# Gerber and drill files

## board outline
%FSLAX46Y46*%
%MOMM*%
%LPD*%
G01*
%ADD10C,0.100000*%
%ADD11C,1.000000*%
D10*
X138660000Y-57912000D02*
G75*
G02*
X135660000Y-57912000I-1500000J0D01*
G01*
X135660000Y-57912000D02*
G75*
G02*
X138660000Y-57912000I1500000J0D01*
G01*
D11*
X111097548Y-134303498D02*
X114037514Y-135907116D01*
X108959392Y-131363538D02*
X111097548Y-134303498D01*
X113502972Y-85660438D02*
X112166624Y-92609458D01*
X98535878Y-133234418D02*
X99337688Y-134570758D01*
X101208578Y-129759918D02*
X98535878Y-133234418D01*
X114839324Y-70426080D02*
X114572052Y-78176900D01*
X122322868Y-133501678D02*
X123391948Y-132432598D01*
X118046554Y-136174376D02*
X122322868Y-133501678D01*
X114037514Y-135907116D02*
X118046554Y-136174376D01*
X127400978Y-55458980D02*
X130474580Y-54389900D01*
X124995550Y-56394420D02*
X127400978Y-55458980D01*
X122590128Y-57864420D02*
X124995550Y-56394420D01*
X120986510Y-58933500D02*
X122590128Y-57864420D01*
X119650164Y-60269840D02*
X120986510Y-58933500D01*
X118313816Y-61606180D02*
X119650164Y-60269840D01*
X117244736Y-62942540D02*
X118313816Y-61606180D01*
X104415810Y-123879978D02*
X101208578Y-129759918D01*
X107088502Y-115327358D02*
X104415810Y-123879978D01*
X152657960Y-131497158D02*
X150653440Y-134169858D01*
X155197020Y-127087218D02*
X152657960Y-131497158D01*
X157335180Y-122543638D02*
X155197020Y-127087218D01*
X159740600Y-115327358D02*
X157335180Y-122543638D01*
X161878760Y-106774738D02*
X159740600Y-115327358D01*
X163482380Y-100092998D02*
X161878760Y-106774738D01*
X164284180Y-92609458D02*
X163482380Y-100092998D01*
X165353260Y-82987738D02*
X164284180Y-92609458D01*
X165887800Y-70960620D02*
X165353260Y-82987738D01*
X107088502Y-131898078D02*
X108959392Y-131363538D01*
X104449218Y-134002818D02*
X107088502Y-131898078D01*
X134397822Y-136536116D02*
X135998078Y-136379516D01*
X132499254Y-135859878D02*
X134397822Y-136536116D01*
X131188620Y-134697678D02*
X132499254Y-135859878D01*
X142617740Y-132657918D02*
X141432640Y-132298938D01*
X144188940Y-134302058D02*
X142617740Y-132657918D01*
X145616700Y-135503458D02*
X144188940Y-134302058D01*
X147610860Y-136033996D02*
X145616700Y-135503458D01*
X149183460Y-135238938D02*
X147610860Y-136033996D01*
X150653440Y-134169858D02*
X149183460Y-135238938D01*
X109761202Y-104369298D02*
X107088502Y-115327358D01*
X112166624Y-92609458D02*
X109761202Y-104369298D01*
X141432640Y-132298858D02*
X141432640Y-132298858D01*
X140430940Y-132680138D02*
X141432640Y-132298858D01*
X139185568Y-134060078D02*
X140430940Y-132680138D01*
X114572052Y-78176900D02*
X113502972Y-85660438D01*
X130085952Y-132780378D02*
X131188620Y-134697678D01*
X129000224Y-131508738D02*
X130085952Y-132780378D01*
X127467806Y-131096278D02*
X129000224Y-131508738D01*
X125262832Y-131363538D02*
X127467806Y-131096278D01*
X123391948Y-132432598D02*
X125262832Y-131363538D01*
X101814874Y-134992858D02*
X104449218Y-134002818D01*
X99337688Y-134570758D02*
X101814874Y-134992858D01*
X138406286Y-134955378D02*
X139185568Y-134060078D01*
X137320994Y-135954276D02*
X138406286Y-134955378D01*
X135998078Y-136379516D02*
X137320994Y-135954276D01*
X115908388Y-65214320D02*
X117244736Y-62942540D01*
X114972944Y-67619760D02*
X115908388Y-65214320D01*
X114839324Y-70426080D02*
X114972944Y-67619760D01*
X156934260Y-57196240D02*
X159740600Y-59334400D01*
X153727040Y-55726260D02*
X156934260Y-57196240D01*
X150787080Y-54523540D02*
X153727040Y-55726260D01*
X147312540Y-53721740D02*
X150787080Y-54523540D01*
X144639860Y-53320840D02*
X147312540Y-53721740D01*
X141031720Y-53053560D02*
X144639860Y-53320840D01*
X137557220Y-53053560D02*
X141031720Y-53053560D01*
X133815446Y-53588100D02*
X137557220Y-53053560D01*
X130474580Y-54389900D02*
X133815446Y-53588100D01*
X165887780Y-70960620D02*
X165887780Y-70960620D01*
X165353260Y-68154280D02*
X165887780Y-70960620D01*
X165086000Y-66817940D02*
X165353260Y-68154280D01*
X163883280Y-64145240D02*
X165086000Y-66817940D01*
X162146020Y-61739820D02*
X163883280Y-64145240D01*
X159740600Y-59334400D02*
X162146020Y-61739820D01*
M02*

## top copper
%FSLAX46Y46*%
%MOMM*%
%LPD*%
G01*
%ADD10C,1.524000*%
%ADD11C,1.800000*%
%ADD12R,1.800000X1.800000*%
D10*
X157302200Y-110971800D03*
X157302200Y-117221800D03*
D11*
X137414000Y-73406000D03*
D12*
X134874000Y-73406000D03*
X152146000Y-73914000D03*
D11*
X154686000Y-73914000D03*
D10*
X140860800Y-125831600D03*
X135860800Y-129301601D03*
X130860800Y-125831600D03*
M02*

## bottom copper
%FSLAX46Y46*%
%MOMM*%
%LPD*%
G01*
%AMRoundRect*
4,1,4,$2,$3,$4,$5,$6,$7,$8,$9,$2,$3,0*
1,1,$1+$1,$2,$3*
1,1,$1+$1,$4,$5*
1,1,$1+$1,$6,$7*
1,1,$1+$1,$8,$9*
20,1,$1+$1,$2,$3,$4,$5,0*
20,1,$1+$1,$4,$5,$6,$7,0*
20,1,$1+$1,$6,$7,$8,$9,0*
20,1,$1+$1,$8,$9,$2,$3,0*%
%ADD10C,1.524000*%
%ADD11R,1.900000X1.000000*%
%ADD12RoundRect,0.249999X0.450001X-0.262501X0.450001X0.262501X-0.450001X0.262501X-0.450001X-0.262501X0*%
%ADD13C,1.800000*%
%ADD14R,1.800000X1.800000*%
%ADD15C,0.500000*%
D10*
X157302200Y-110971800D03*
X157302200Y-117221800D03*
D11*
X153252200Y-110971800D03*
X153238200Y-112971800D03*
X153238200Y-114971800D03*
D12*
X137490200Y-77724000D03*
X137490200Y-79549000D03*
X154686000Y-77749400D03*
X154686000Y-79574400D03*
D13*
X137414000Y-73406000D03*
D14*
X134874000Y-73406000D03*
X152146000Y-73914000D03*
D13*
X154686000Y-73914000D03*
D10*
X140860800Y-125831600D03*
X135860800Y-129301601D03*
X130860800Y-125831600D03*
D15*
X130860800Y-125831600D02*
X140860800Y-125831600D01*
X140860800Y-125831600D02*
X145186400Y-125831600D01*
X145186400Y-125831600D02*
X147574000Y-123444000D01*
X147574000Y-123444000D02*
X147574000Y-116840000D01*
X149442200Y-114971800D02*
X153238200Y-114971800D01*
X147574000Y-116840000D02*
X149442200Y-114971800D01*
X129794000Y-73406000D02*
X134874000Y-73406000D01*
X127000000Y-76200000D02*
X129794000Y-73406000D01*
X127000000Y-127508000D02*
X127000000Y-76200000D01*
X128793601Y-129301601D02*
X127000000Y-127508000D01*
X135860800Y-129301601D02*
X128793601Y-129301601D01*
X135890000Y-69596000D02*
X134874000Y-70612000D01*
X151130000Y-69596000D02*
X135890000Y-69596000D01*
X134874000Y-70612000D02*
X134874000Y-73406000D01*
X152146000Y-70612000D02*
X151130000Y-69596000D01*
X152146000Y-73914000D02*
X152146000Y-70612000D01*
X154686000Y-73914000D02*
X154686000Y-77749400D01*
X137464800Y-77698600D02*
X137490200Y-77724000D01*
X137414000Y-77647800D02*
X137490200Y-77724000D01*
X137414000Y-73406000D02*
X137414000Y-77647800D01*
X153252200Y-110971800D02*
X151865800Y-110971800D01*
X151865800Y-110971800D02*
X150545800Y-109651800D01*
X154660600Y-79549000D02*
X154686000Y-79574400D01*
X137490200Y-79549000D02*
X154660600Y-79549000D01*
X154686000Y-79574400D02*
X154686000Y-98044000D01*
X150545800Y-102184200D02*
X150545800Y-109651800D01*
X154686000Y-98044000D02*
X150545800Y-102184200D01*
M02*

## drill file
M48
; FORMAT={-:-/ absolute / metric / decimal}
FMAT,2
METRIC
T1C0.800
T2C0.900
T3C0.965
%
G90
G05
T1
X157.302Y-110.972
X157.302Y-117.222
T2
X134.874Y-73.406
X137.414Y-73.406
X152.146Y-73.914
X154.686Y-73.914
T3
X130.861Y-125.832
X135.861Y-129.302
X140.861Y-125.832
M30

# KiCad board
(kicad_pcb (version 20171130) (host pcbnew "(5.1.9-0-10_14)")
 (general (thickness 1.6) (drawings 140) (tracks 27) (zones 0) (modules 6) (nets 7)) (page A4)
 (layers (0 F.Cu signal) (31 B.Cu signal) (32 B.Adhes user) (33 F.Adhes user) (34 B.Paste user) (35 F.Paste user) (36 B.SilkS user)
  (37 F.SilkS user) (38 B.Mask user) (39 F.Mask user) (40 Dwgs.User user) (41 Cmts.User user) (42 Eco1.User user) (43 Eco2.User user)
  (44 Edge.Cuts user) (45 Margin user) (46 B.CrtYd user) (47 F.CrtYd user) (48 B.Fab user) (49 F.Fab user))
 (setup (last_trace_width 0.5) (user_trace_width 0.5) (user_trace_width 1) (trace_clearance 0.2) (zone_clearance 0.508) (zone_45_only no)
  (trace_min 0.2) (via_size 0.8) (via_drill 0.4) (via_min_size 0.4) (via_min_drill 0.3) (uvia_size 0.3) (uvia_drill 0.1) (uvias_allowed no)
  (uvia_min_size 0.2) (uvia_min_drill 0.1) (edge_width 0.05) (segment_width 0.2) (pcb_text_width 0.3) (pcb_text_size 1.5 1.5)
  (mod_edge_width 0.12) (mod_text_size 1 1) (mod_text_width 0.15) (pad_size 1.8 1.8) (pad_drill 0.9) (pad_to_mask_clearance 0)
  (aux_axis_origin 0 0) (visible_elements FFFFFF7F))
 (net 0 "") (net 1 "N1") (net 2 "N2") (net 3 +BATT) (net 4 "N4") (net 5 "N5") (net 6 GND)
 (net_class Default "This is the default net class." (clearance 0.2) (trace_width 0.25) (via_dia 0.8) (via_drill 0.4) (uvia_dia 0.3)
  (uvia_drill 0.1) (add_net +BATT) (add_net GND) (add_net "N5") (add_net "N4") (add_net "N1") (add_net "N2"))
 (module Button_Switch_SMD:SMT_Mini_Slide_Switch (layer B.Cu) (at 155.0162 114.0968 270)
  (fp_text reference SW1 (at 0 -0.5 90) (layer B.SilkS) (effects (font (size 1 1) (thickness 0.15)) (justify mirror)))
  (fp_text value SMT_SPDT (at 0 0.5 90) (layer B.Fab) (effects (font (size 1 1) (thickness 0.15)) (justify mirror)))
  (pad "" thru_hole circle (at -3.125 -2.286 270) (size 1.524 1.524) (drill 0.8) (layers *.Cu *.Mask))
  (pad "" thru_hole circle (at 3.125 -2.286 270) (size 1.524 1.524) (drill 0.8) (layers *.Cu *.Mask))
  (pad 1 smd rect (at -3.125 1.764 270) (size 1 1.9) (layers B.Cu B.Paste B.Mask) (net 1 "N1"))
  (pad 2 smd rect (at -1.125 1.778 270) (size 1 1.9) (layers B.Cu B.Paste B.Mask) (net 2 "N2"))
  (pad 3 smd rect (at 0.875 1.778 270) (size 1 1.9) (layers B.Cu B.Paste B.Mask) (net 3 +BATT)))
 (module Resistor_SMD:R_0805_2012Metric (layer B.Cu) (at 137.4902 78.6365 90)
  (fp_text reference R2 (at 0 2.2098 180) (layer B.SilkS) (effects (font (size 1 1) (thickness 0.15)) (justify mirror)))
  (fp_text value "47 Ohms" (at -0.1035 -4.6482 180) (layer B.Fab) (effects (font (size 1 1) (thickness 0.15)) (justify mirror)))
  (pad 2 smd roundrect (at 0.9125 0 90) (size 1.025 1.4) (layers B.Cu B.Paste B.Mask) (roundrect_rratio 0.2439014634146341) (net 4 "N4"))
  (pad 1 smd roundrect (at -0.9125 0 90) (size 1.025 1.4) (layers B.Cu B.Paste B.Mask) (roundrect_rratio 0.2439014634146341) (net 1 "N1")))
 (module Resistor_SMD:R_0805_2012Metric (layer B.Cu) (at 154.686 78.6619 90)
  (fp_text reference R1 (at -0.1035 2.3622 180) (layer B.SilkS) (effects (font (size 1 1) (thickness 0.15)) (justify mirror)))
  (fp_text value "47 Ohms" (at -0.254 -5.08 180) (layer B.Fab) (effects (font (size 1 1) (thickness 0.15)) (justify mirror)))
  (pad 2 smd roundrect (at 0.9125 0 90) (size 1.025 1.4) (layers B.Cu B.Paste B.Mask) (roundrect_rratio 0.2439014634146341) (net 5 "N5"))
  (pad 1 smd roundrect (at -0.9125 0 90) (size 1.025 1.4) (layers B.Cu B.Paste B.Mask) (roundrect_rratio 0.2439014634146341) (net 1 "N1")))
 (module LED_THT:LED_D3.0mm (layer F.Cu) (at 134.874 73.406)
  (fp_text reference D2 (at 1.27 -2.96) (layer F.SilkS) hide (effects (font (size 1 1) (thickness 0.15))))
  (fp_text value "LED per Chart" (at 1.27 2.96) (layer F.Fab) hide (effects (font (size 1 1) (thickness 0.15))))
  (pad 2 thru_hole circle (at 2.54 0) (size 1.8 1.8) (drill 0.9) (layers *.Cu *.Mask) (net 4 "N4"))
  (pad 1 thru_hole rect (at 0 0) (size 1.8 1.8) (drill 0.9) (layers *.Cu *.Mask) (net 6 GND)))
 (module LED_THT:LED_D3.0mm (layer F.Cu) (at 152.146 73.914)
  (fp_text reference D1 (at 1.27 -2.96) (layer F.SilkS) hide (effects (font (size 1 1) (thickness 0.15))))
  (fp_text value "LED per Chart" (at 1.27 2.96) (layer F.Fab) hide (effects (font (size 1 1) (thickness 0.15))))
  (pad 1 thru_hole rect (at 0 0) (size 1.8 1.8) (drill 0.9) (layers *.Cu *.Mask) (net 6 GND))
  (pad 2 thru_hole circle (at 2.54 0) (size 1.8 1.8) (drill 0.9) (layers *.Cu *.Mask) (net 5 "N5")))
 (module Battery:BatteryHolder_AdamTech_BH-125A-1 (layer B.Cu) (at 130.8608 125.8316)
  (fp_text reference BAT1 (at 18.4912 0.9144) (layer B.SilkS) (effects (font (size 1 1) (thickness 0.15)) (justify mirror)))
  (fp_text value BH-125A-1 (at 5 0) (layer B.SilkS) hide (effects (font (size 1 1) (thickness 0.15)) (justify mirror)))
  (pad POS2 thru_hole circle (at 10 0) (size 1.524 1.524) (drill 0.9652) (layers *.Cu *.Mask) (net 3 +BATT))
  (pad NEG thru_hole circle (at 5 3.470001) (size 1.524 1.524) (drill 0.9652) (layers *.Cu *.Mask) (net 6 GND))
  (pad POS1 thru_hole circle (at 0 0) (size 1.524 1.524) (drill 0.9652) (layers *.Cu *.Mask) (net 3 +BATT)))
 (gr_circle (center 137.16 57.912) (end 138.66 57.912) (layer Edge.Cuts) (width 0.1))
 (gr_line (start 111.097548 134.303498) (end 114.037514 135.907116) (layer Edge.Cuts) (width 1))
 (gr_line (start 108.959392 131.363538) (end 111.097548 134.303498) (layer Edge.Cuts) (width 1))
 (gr_line (start 113.502972 85.660438) (end 112.166624 92.609458) (layer Edge.Cuts) (width 1))
 (gr_line (start 98.535878 133.234418) (end 99.337688 134.570758) (layer Edge.Cuts) (width 1))
 (gr_line (start 101.208578 129.759918) (end 98.535878 133.234418) (layer Edge.Cuts) (width 1))
 (gr_line (start 114.839324 70.42608) (end 114.572052 78.1769) (layer Edge.Cuts) (width 1))
 (gr_line (start 122.322868 133.501678) (end 123.391948 132.432598) (layer Edge.Cuts) (width 1))
 (gr_line (start 118.046554 136.174376) (end 122.322868 133.501678) (layer Edge.Cuts) (width 1))
 (gr_line (start 114.037514 135.907116) (end 118.046554 136.174376) (layer Edge.Cuts) (width 1))
 (gr_line (start 127.400978 55.45898) (end 130.47458 54.3899) (layer Edge.Cuts) (width 1))
 (gr_line (start 124.99555 56.39442) (end 127.400978 55.45898) (layer Edge.Cuts) (width 1))
 (gr_line (start 122.590128 57.86442) (end 124.99555 56.39442) (layer Edge.Cuts) (width 1))
 (gr_line (start 120.98651 58.9335) (end 122.590128 57.86442) (layer Edge.Cuts) (width 1))
 (gr_line (start 119.650164 60.26984) (end 120.98651 58.9335) (layer Edge.Cuts) (width 1))
 (gr_line (start 118.313816 61.60618) (end 119.650164 60.26984) (layer Edge.Cuts) (width 1))
 (gr_line (start 117.244736 62.94254) (end 118.313816 61.60618) (layer Edge.Cuts) (width 1))
 (gr_line (start 104.41581 123.879978) (end 101.208578 129.759918) (layer Edge.Cuts) (width 1))
 (gr_line (start 107.088502 115.327358) (end 104.41581 123.879978) (layer Edge.Cuts) (width 1))
 (gr_line (start 152.65796 131.497158) (end 150.65344 134.169858) (layer Edge.Cuts) (width 1))
 (gr_line (start 155.19702 127.087218) (end 152.65796 131.497158) (layer Edge.Cuts) (width 1))
 (gr_line (start 157.33518 122.543638) (end 155.19702 127.087218) (layer Edge.Cuts) (width 1))
 (gr_line (start 159.7406 115.327358) (end 157.33518 122.543638) (layer Edge.Cuts) (width 1))
 (gr_line (start 161.87876 106.774738) (end 159.7406 115.327358) (layer Edge.Cuts) (width 1))
 (gr_line (start 163.48238 100.092998) (end 161.87876 106.774738) (layer Edge.Cuts) (width 1))
 (gr_line (start 164.28418 92.609458) (end 163.48238 100.092998) (layer Edge.Cuts) (width 1))
 (gr_line (start 165.35326 82.987738) (end 164.28418 92.609458) (layer Edge.Cuts) (width 1))
 (gr_line (start 165.8878 70.96062) (end 165.35326 82.987738) (layer Edge.Cuts) (width 1))
 (gr_line (start 107.088502 131.898078) (end 108.959392 131.363538) (layer Edge.Cuts) (width 1))
 (gr_line (start 104.449218 134.002818) (end 107.088502 131.898078) (layer Edge.Cuts) (width 1))
 (gr_line (start 134.397822 136.536116) (end 135.998078 136.379516) (layer Edge.Cuts) (width 1))
 (gr_line (start 132.499254 135.859878) (end 134.397822 136.536116) (layer Edge.Cuts) (width 1))
 (gr_line (start 131.18862 134.697678) (end 132.499254 135.859878) (layer Edge.Cuts) (width 1))
 (gr_line (start 142.61774 132.657918) (end 141.43264 132.298938) (layer Edge.Cuts) (width 1))
 (gr_line (start 144.18894 134.302058) (end 142.61774 132.657918) (layer Edge.Cuts) (width 1))
 (gr_line (start 145.6167 135.503458) (end 144.18894 134.302058) (layer Edge.Cuts) (width 1))
 (gr_line (start 147.61086 136.033996) (end 145.6167 135.503458) (layer Edge.Cuts) (width 1))
 (gr_line (start 149.18346 135.238938) (end 147.61086 136.033996) (layer Edge.Cuts) (width 1))
 (gr_line (start 150.65344 134.169858) (end 149.18346 135.238938) (layer Edge.Cuts) (width 1))
 (gr_line (start 109.761202 104.369298) (end 107.088502 115.327358) (layer Edge.Cuts) (width 1))
 (gr_line (start 112.166624 92.609458) (end 109.761202 104.369298) (layer Edge.Cuts) (width 1))
 (gr_line (start 141.43264 132.298858) (end 141.43264 132.298858) (layer Edge.Cuts) (width 1))
 (gr_line (start 140.43094 132.680138) (end 141.43264 132.298858) (layer Edge.Cuts) (width 1))
 (gr_line (start 139.185568 134.060078) (end 140.43094 132.680138) (layer Edge.Cuts) (width 1))
 (gr_line (start 114.572052 78.1769) (end 113.502972 85.660438) (layer Edge.Cuts) (width 1))
 (gr_line (start 130.085952 132.780378) (end 131.18862 134.697678) (layer Edge.Cuts) (width 1))
 (gr_line (start 129.000224 131.508738) (end 130.085952 132.780378) (layer Edge.Cuts) (width 1))
 (gr_line (start 127.467806 131.096278) (end 129.000224 131.508738) (layer Edge.Cuts) (width 1))
 (gr_line (start 125.262832 131.363538) (end 127.467806 131.096278) (layer Edge.Cuts) (width 1))
 (gr_line (start 123.391948 132.432598) (end 125.262832 131.363538) (layer Edge.Cuts) (width 1))
 (gr_line (start 101.814874 134.992858) (end 104.449218 134.002818) (layer Edge.Cuts) (width 1))
 (gr_line (start 99.337688 134.570758) (end 101.814874 134.992858) (layer Edge.Cuts) (width 1))
 (gr_line (start 138.406286 134.955378) (end 139.185568 134.060078) (layer Edge.Cuts) (width 1))
 (gr_line (start 137.320994 135.954276) (end 138.406286 134.955378) (layer Edge.Cuts) (width 1))
 (gr_line (start 135.998078 136.379516) (end 137.320994 135.954276) (layer Edge.Cuts) (width 1))
 (gr_line (start 115.908388 65.21432) (end 117.244736 62.94254) (layer Edge.Cuts) (width 1))
 (gr_line (start 114.972944 67.61976) (end 115.908388 65.21432) (layer Edge.Cuts) (width 1))
 (gr_line (start 114.839324 70.42608) (end 114.972944 67.61976) (layer Edge.Cuts) (width 1))
 (gr_line (start 156.93426 57.19624) (end 159.7406 59.3344) (layer Edge.Cuts) (width 1))
 (gr_line (start 153.72704 55.72626) (end 156.93426 57.19624) (layer Edge.Cuts) (width 1))
 (gr_line (start 150.78708 54.52354) (end 153.72704 55.72626) (layer Edge.Cuts) (width 1))
 (gr_line (start 147.31254 53.72174) (end 150.78708 54.52354) (layer Edge.Cuts) (width 1))
 (gr_line (start 144.63986 53.32084) (end 147.31254 53.72174) (layer Edge.Cuts) (width 1))
 (gr_line (start 141.03172 53.05356) (end 144.63986 53.32084) (layer Edge.Cuts) (width 1))
 (gr_line (start 137.55722 53.05356) (end 141.03172 53.05356) (layer Edge.Cuts) (width 1))
 (gr_line (start 133.815446 53.5881) (end 137.55722 53.05356) (layer Edge.Cuts) (width 1))
 (gr_line (start 130.47458 54.3899) (end 133.815446 53.5881) (layer Edge.Cuts) (width 1))
 (gr_line (start 165.88778 70.96062) (end 165.88778 70.96062) (layer Edge.Cuts) (width 1))
 (gr_line (start 165.35326 68.15428) (end 165.88778 70.96062) (layer Edge.Cuts) (width 1))
 (gr_line (start 165.086 66.81794) (end 165.35326 68.15428) (layer Edge.Cuts) (width 1))
 (gr_line (start 163.88328 64.14524) (end 165.086 66.81794) (layer Edge.Cuts) (width 1))
 (gr_line (start 162.14602 61.73982) (end 163.88328 64.14524) (layer Edge.Cuts) (width 1))
 (gr_line (start 159.7406 59.3344) (end 162.14602 61.73982) (layer Edge.Cuts) (width 1))
 (segment (start 130.8608 125.8316) (end 140.8608 125.8316) (width 0.5) (layer B.Cu) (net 3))
 (segment (start 140.8608 125.8316) (end 145.1864 125.8316) (width 0.5) (layer B.Cu) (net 3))
 (segment (start 145.1864 125.8316) (end 147.574 123.444) (width 0.5) (layer B.Cu) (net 3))
 (segment (start 147.574 123.444) (end 147.574 116.84) (width 0.5) (layer B.Cu) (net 3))
 (segment (start 149.4422 114.9718) (end 153.2382 114.9718) (width 0.5) (layer B.Cu) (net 3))
 (segment (start 147.574 116.84) (end 149.4422 114.9718) (width 0.5) (layer B.Cu) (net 3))
 (segment (start 129.794 73.406) (end 134.874 73.406) (width 0.5) (layer B.Cu) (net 6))
 (segment (start 127 76.2) (end 129.794 73.406) (width 0.5) (layer B.Cu) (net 6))
 (segment (start 127 127.508) (end 127 76.2) (width 0.5) (layer B.Cu) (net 6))
 (segment (start 128.793601 129.301601) (end 127 127.508) (width 0.5) (layer B.Cu) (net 6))
 (segment (start 135.8608 129.301601) (end 128.793601 129.301601) (width 0.5) (layer B.Cu) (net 6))
 (segment (start 135.89 69.596) (end 134.874 70.612) (width 0.5) (layer B.Cu) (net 6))
 (segment (start 151.13 69.596) (end 135.89 69.596) (width 0.5) (layer B.Cu) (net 6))
 (segment (start 134.874 70.612) (end 134.874 73.406) (width 0.5) (layer B.Cu) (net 6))
 (segment (start 152.146 70.612) (end 151.13 69.596) (width 0.5) (layer B.Cu) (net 6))
 (segment (start 152.146 73.914) (end 152.146 70.612) (width 0.5) (layer B.Cu) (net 6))
 (segment (start 154.686 73.914) (end 154.686 77.7494) (width 0.5) (layer B.Cu) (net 5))
 (segment (start 137.4648 77.6986) (end 137.4902 77.724) (width 0.5) (layer B.Cu) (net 4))
 (segment (start 137.414 77.6478) (end 137.4902 77.724) (width 0.5) (layer B.Cu) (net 4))
 (segment (start 137.414 73.406) (end 137.414 77.6478) (width 0.5) (layer B.Cu) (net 4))
 (segment (start 153.2522 110.9718) (end 151.8658 110.9718) (width 0.5) (layer B.Cu) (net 1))
 (segment (start 151.8658 110.9718) (end 150.5458 109.6518) (width 0.5) (layer B.Cu) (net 1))
 (segment (start 154.6606 79.549) (end 154.686 79.5744) (width 0.5) (layer B.Cu) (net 1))
 (segment (start 137.4902 79.549) (end 154.6606 79.549) (width 0.5) (layer B.Cu) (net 1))
 (segment (start 154.686 79.5744) (end 154.686 98.044) (width 0.5) (layer B.Cu) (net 1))
 (segment (start 150.5458 102.1842) (end 150.5458 109.6518) (width 0.5) (layer B.Cu) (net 1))
 (segment (start 154.686 98.044) (end 150.5458 102.1842) (width 0.5) (layer B.Cu) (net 1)))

